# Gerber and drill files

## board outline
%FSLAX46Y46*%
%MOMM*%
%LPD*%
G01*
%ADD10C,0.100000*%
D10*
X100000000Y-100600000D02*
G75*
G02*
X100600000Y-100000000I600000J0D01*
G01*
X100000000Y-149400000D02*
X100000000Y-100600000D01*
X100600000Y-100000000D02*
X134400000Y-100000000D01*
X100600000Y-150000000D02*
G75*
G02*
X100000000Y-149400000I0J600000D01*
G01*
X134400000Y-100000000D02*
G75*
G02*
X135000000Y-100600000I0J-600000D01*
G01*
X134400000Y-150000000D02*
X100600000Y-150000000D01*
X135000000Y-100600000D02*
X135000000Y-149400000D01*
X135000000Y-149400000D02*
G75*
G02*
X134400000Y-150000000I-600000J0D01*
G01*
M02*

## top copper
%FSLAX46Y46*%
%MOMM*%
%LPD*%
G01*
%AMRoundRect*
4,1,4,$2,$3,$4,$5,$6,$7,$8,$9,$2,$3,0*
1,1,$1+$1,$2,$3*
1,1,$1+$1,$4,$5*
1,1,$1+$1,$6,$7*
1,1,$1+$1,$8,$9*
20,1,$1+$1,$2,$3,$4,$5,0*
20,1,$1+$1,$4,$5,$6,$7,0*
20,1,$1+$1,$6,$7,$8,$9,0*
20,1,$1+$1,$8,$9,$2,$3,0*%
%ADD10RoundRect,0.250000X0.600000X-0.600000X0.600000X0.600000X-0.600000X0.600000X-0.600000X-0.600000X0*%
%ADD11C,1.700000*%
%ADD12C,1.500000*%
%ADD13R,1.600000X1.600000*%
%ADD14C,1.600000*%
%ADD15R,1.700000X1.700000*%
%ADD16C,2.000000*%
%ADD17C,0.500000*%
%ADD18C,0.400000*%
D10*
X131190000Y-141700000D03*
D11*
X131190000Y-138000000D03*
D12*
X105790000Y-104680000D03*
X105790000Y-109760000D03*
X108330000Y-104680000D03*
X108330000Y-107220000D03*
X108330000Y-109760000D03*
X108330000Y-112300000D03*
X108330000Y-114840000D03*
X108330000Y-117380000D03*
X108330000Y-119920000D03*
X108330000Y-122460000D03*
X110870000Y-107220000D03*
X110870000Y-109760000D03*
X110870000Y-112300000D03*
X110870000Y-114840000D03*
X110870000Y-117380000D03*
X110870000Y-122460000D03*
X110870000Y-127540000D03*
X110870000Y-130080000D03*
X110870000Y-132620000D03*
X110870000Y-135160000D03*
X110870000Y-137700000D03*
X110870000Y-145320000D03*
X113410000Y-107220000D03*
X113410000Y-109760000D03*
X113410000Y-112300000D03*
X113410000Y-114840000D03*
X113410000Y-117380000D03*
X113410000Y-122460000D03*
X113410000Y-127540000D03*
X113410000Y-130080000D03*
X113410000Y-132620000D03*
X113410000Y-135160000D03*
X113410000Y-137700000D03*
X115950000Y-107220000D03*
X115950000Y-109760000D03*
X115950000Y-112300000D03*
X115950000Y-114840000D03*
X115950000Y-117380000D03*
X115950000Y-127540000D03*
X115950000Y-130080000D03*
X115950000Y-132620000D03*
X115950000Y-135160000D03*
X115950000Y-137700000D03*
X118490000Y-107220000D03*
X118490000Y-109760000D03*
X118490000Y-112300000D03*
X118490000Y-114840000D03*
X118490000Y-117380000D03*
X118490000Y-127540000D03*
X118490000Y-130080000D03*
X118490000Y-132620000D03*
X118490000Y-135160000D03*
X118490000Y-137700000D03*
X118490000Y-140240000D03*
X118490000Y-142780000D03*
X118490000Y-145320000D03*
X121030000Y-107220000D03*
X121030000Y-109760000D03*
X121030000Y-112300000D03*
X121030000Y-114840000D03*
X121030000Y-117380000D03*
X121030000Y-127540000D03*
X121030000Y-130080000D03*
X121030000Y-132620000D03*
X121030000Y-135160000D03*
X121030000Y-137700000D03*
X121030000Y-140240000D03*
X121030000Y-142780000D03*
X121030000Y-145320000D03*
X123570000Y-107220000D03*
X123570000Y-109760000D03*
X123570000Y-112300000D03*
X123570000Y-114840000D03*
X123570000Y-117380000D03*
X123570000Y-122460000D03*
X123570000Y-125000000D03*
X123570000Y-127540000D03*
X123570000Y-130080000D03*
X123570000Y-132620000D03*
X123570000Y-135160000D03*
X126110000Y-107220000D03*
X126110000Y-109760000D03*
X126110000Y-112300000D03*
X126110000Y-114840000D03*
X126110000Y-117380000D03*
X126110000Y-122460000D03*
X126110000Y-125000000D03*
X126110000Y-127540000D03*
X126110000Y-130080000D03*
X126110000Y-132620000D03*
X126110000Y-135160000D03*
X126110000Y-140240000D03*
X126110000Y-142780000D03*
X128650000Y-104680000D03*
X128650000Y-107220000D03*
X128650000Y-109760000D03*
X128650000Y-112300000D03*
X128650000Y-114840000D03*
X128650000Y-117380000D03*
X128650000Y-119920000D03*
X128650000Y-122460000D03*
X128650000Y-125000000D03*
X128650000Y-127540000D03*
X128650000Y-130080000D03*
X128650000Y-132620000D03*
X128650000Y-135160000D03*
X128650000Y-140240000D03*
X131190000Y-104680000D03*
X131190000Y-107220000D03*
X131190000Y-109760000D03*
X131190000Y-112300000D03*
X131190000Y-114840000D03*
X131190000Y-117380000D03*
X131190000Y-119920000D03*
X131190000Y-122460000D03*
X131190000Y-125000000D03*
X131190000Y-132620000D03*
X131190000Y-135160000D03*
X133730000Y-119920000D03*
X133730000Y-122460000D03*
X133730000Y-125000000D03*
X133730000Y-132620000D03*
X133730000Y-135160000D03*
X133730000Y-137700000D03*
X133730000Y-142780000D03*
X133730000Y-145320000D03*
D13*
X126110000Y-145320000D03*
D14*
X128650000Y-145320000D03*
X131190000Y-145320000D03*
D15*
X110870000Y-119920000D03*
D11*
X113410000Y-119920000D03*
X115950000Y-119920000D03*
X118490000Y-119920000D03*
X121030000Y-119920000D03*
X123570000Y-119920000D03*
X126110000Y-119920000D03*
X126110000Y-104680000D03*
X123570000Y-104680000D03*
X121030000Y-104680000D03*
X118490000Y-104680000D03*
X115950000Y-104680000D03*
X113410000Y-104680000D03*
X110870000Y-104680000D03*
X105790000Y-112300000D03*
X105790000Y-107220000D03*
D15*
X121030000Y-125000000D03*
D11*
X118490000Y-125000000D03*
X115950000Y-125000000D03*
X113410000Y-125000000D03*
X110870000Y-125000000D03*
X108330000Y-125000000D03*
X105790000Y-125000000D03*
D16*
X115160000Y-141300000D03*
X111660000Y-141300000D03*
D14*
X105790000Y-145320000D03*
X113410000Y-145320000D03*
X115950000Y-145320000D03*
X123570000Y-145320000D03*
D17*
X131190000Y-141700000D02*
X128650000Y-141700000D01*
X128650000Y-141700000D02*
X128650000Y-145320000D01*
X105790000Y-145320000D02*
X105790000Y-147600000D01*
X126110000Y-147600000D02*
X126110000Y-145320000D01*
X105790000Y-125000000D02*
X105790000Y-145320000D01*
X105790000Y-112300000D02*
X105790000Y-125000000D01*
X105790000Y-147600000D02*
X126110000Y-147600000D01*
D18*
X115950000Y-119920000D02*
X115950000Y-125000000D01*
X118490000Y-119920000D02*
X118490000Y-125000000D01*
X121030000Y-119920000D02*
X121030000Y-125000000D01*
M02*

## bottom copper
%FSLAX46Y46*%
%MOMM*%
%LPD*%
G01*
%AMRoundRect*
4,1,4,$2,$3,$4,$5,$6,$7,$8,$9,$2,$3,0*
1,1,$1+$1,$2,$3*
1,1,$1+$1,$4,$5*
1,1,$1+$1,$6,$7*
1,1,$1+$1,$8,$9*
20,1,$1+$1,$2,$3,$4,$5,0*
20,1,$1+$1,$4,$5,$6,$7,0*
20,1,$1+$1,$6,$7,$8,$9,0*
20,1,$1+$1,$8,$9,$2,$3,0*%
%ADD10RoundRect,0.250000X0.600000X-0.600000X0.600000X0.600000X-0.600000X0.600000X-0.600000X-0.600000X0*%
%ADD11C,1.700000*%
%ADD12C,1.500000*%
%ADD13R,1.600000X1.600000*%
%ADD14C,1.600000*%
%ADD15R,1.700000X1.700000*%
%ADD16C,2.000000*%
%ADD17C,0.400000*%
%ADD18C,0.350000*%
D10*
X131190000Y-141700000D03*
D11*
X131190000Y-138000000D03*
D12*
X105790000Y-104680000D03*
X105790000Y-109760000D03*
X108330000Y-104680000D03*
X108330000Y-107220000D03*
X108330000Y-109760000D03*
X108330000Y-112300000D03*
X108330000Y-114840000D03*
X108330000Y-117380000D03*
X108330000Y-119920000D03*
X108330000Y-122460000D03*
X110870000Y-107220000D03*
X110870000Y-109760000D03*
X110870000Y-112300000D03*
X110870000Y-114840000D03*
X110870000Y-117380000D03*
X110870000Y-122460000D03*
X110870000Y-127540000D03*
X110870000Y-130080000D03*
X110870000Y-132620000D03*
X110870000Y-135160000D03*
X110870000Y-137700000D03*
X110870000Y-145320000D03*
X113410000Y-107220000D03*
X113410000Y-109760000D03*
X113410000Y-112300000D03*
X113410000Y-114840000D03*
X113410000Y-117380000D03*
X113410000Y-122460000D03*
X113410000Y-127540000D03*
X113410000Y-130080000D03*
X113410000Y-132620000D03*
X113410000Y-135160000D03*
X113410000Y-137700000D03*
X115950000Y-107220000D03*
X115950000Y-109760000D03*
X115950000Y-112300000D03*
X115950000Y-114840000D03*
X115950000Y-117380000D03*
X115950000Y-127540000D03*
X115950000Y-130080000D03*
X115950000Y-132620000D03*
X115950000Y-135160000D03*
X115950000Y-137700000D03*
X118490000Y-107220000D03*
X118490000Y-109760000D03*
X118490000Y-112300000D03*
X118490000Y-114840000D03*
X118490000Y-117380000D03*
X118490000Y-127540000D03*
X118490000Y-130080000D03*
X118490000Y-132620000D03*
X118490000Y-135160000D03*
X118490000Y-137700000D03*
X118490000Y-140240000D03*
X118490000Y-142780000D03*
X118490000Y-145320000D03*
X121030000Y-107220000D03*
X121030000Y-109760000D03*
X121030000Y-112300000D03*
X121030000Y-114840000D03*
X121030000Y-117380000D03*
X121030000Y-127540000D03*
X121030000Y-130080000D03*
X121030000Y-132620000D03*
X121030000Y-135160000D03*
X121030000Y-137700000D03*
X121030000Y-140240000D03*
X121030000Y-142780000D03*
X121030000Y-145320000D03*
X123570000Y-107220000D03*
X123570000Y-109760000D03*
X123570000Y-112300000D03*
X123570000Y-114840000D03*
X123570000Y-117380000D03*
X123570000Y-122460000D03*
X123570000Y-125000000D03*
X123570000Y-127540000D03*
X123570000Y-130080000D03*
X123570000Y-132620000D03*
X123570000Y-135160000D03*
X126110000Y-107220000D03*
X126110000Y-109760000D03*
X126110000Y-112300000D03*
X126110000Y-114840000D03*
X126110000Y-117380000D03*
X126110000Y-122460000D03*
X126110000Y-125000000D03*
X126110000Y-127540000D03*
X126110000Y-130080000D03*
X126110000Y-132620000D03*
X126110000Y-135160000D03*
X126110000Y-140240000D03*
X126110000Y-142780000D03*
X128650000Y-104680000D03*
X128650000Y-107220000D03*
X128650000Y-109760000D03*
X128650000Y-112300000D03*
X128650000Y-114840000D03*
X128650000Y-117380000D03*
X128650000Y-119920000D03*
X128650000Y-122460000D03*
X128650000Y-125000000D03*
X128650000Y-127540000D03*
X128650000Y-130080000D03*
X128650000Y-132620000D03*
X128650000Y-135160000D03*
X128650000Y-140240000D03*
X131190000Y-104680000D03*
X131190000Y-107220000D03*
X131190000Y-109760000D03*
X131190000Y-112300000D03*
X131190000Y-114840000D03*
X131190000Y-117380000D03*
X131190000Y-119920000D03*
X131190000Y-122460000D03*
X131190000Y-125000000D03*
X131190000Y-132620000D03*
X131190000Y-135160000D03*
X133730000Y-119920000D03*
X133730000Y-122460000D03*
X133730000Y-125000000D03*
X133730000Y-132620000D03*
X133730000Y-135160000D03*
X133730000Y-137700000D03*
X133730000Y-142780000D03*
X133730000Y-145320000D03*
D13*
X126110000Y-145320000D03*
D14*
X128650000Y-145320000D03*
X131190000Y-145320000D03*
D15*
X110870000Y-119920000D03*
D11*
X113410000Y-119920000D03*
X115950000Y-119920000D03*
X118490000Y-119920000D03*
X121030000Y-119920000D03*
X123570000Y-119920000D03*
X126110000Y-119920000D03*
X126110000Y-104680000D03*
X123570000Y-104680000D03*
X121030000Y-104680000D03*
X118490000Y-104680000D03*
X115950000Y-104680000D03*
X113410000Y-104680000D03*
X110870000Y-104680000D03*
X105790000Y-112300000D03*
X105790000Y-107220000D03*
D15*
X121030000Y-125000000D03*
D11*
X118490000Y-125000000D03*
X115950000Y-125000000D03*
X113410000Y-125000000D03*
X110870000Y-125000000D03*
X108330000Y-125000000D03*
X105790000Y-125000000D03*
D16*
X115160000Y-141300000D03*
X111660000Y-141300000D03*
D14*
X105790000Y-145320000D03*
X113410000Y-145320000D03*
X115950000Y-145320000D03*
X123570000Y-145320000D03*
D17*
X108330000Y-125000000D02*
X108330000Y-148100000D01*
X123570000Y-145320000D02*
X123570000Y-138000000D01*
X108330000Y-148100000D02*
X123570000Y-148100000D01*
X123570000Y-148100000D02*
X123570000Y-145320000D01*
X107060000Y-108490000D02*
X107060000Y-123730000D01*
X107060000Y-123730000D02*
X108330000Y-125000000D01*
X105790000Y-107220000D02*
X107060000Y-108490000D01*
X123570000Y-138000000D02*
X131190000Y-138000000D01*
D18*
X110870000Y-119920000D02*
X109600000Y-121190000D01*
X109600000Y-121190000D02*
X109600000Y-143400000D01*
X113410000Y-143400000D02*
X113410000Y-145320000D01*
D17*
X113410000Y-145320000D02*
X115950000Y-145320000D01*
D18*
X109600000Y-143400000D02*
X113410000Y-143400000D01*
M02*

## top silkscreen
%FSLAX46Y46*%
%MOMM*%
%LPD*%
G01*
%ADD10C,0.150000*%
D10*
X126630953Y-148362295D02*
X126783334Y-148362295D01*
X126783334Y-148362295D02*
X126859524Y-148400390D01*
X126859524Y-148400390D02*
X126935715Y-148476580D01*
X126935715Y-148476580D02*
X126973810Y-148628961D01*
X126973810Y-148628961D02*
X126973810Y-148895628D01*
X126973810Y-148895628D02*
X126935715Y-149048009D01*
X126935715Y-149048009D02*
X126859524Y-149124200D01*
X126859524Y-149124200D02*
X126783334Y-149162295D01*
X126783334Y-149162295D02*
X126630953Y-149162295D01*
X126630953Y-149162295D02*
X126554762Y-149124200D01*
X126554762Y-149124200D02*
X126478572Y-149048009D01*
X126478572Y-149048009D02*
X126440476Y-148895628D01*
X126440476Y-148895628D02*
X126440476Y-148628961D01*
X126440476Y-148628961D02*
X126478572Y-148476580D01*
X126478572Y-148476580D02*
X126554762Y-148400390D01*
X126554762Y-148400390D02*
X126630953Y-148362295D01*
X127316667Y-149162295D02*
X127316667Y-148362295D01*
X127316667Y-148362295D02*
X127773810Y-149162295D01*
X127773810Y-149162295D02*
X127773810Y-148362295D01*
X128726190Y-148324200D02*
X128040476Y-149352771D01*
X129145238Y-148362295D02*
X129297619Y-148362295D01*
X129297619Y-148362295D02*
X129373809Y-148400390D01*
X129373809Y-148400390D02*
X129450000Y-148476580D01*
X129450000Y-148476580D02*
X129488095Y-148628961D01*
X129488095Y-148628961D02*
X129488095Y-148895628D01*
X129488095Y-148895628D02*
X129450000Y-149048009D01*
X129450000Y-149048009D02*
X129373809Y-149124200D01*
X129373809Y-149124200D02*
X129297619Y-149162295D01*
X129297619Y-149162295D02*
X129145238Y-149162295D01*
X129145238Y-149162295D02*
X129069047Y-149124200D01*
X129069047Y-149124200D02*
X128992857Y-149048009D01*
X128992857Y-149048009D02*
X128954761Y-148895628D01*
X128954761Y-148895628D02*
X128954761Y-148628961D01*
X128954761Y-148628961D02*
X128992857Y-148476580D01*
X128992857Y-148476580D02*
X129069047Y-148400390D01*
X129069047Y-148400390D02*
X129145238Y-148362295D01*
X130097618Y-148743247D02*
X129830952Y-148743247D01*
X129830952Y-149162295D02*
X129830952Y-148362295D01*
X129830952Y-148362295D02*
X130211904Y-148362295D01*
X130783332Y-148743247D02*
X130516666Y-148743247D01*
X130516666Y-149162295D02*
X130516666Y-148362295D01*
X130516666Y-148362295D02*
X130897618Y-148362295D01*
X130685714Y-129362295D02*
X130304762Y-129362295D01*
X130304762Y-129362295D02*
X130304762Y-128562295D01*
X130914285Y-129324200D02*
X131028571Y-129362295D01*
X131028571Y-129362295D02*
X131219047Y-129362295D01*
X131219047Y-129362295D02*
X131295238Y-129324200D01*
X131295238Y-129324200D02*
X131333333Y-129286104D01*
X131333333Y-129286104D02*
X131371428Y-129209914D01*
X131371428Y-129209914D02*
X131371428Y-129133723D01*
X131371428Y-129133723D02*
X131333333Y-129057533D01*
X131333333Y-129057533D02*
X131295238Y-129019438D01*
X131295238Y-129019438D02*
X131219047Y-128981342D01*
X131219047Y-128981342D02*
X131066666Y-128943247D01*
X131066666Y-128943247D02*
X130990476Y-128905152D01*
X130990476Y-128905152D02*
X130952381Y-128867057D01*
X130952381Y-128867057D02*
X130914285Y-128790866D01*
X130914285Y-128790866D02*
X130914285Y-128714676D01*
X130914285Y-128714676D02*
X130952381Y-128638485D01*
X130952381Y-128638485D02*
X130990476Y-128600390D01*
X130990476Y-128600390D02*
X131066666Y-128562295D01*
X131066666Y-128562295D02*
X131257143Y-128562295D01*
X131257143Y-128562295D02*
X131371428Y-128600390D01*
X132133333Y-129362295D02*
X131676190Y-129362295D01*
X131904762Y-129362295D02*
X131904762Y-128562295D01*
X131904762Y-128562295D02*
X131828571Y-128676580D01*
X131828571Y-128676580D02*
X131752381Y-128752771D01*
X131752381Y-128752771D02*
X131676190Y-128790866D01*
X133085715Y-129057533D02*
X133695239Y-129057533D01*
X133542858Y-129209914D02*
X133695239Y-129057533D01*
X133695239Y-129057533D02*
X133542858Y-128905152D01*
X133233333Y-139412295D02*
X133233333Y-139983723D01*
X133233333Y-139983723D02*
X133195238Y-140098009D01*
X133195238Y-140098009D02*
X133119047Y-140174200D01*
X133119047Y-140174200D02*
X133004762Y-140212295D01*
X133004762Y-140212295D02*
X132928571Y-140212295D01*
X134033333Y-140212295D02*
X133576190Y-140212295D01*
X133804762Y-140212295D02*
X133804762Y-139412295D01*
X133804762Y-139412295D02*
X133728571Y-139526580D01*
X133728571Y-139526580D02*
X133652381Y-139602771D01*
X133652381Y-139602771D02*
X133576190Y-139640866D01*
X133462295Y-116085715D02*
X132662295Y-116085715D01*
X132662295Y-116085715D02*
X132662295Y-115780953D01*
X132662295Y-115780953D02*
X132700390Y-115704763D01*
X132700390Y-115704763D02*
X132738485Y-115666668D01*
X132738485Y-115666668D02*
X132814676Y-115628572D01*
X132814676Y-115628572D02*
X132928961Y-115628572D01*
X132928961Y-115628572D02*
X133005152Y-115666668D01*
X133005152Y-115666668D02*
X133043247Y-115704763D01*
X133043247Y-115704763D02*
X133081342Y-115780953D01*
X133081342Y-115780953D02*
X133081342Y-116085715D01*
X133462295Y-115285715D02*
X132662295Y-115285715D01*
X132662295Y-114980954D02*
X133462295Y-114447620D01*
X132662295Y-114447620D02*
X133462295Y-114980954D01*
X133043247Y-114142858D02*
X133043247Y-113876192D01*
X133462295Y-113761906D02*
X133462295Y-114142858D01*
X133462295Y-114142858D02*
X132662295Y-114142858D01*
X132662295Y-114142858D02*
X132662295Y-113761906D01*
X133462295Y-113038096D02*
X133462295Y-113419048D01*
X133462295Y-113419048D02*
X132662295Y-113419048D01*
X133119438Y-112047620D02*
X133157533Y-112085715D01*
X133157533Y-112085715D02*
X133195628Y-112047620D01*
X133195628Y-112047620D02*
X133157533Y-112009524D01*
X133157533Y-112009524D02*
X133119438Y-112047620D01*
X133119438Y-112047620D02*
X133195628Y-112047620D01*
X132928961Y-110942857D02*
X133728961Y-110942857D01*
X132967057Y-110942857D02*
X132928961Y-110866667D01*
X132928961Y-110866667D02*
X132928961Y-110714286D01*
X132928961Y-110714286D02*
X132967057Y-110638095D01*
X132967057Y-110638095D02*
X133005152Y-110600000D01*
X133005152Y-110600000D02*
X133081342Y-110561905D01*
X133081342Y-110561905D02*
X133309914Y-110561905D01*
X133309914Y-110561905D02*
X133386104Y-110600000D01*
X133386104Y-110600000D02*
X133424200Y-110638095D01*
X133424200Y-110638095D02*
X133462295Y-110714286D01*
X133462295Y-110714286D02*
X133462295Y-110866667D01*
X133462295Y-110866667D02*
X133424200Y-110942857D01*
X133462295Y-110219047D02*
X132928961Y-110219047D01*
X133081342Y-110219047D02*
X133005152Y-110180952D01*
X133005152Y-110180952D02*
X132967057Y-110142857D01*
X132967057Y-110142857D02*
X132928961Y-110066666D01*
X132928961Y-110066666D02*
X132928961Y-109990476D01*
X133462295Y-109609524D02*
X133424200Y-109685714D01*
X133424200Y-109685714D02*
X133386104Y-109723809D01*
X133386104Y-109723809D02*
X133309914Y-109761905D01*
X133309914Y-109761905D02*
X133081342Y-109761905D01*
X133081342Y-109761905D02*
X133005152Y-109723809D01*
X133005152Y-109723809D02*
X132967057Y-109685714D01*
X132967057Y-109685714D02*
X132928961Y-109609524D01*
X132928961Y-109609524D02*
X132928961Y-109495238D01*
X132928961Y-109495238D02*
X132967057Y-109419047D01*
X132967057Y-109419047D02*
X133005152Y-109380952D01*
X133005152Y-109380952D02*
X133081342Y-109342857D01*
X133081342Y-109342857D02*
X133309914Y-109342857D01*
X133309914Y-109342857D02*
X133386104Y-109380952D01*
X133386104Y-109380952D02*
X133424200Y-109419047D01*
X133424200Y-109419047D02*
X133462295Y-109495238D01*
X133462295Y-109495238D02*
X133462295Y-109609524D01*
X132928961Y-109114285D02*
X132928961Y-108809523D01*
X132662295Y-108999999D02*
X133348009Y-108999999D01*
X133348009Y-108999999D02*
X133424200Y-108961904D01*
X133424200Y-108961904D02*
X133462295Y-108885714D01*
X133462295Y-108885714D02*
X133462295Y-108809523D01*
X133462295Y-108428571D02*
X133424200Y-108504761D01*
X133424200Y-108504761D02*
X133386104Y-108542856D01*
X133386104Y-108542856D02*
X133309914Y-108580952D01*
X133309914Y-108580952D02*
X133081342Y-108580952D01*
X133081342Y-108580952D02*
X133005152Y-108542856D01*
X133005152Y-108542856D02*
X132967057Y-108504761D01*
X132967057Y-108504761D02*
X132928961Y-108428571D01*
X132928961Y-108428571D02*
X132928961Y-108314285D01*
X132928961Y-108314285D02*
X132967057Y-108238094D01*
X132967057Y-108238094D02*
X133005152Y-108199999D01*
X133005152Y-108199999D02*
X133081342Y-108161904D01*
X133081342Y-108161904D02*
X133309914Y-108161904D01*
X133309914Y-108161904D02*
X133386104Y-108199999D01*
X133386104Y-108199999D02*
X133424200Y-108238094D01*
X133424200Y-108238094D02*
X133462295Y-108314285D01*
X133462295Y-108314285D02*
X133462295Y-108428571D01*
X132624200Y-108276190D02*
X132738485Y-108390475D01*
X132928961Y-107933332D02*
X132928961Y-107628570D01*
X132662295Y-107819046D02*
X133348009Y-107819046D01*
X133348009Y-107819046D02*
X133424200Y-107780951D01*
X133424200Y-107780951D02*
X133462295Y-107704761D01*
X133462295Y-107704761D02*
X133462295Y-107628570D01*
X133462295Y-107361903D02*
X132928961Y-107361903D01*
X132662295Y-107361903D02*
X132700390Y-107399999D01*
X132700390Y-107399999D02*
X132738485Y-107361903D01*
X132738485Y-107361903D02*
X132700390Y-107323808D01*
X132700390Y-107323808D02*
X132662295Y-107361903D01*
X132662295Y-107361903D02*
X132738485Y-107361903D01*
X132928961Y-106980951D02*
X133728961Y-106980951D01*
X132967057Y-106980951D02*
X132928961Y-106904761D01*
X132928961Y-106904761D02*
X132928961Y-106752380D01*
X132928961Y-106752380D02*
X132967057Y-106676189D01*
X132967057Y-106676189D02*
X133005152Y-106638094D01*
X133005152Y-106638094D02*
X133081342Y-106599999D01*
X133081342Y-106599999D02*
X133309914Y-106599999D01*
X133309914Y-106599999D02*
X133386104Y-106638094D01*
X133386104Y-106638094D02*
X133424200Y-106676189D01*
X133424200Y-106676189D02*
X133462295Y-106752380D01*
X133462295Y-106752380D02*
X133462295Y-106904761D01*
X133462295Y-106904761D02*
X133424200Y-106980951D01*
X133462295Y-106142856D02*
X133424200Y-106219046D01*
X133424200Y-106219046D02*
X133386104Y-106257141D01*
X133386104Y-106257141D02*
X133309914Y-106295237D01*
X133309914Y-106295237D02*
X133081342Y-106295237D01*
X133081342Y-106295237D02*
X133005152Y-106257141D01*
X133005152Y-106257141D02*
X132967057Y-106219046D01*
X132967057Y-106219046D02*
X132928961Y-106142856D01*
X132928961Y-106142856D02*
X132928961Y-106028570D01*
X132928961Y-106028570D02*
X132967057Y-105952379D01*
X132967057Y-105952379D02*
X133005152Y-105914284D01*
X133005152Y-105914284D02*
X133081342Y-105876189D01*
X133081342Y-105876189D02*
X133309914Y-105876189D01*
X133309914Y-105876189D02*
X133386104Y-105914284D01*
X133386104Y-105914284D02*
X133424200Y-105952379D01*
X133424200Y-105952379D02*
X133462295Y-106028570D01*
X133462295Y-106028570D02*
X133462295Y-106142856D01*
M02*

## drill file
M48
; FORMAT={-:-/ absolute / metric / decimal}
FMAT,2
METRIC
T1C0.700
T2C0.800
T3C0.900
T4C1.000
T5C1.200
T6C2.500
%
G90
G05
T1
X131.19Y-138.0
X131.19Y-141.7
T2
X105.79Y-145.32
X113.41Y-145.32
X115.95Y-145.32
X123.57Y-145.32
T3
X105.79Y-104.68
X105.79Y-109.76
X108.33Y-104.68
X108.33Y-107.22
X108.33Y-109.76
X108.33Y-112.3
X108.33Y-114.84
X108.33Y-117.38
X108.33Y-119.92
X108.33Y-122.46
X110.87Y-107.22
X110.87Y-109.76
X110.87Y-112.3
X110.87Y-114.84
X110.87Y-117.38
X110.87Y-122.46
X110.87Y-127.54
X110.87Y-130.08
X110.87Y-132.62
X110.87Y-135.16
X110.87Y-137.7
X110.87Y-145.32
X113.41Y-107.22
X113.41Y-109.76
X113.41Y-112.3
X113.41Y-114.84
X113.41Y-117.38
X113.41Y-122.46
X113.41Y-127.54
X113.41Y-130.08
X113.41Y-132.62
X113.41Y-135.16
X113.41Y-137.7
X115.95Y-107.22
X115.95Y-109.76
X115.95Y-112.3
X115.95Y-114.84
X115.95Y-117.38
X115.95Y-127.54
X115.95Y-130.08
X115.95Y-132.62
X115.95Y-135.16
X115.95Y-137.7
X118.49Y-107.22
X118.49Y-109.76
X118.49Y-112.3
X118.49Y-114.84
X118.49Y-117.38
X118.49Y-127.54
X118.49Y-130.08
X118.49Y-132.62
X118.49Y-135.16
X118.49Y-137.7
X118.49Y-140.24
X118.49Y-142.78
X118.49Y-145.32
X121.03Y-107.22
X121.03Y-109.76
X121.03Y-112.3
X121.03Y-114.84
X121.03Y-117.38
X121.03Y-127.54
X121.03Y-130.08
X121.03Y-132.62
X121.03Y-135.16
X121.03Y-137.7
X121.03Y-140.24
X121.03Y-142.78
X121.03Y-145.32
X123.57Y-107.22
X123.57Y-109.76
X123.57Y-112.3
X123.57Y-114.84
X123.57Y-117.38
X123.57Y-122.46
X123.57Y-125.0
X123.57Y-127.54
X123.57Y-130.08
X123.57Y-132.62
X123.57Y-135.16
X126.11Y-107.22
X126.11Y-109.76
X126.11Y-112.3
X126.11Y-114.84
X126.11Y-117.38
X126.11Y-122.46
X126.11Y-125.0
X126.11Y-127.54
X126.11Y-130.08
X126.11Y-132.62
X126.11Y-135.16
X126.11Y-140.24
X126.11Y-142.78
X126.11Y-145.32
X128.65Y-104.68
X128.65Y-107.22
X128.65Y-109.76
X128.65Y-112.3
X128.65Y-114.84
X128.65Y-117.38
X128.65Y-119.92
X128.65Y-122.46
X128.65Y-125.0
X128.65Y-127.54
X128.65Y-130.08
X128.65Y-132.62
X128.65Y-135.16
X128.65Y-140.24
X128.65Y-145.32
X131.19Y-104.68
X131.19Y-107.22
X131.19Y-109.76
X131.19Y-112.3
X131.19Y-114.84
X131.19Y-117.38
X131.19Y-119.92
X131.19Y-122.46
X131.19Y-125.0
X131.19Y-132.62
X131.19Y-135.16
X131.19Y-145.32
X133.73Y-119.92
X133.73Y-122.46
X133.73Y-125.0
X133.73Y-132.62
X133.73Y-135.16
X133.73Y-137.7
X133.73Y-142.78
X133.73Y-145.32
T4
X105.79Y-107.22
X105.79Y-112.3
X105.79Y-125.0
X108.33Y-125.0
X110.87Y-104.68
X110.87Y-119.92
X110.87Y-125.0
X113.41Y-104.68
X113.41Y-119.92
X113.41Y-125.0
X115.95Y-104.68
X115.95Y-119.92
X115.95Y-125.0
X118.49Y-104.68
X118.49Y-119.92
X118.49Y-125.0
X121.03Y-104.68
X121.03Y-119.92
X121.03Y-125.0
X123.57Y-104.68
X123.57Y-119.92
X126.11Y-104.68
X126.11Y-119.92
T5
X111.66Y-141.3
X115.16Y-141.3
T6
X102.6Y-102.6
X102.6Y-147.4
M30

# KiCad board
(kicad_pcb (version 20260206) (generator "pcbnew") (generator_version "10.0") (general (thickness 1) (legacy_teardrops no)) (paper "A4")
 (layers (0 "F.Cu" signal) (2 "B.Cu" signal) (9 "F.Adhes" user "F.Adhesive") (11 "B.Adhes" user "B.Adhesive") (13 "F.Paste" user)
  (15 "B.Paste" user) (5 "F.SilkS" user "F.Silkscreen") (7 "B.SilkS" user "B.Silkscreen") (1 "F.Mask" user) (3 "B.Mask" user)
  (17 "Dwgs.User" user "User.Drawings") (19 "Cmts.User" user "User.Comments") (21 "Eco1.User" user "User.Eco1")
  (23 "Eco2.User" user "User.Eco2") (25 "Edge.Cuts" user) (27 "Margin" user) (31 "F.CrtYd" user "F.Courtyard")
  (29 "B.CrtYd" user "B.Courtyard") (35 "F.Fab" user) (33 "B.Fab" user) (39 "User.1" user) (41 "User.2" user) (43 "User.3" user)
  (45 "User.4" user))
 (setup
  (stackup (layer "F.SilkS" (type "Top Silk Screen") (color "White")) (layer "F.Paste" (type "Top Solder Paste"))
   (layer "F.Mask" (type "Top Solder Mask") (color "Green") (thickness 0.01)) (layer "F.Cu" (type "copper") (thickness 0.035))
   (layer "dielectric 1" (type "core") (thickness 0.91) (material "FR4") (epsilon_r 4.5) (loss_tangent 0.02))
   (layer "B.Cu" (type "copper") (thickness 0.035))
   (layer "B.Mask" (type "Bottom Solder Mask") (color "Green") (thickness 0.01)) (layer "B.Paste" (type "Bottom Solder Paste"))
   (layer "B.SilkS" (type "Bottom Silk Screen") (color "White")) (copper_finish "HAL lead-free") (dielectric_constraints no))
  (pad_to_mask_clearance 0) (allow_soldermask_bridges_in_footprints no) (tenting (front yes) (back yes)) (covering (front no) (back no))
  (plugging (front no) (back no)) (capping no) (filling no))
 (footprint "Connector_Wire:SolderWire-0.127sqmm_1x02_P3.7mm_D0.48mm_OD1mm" (layer "F.Cu") (at 131.19 141.7 90)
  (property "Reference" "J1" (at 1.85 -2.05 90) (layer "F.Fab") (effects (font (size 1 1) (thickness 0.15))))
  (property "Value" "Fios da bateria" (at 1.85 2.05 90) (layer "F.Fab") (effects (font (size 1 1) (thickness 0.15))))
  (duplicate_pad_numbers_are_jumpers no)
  (pad "1" thru_hole roundrect (at 0 0 90) (size 1.7 1.7) (drill 0.7) (layers "*.Cu" "*.Mask") (remove_unused_layers no)
   (roundrect_rratio 0.147059) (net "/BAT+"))
  (pad "2" thru_hole circle (at 3.7 0 90) (size 1.7 1.7) (drill 0.7) (layers "*.Cu" "*.Mask") (remove_unused_layers no) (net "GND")))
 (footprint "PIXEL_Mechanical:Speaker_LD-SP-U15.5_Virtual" (layer "F.Cu") (at 143.7 129)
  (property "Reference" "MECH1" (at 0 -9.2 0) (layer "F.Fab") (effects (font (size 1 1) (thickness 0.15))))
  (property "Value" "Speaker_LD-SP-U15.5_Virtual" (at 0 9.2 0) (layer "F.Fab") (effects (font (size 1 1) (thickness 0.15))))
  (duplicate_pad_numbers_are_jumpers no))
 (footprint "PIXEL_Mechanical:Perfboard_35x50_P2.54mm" (layer "F.Cu") (at 0 0)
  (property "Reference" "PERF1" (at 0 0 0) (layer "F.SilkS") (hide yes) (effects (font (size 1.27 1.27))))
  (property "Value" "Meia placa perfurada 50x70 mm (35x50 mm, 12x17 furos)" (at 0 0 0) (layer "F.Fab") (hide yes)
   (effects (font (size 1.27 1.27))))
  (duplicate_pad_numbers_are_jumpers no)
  (pad "" np_thru_hole circle (at 102.6 102.6) (size 2.5 2.5) (drill 2.5) (layers "*.Cu" "*.Mask"))
  (pad "" np_thru_hole circle (at 102.6 147.4) (size 2.5 2.5) (drill 2.5) (layers "*.Cu" "*.Mask"))
  (pad "" thru_hole circle (at 105.79 104.68) (size 1.5 1.5) (drill 0.9) (layers "*.Cu" "*.Mask") (remove_unused_layers no))
  (pad "" thru_hole circle (at 105.79 109.76) (size 1.5 1.5) (drill 0.9) (layers "*.Cu" "*.Mask") (remove_unused_layers no))
  (pad "" thru_hole circle (at 108.33 104.68) (size 1.5 1.5) (drill 0.9) (layers "*.Cu" "*.Mask") (remove_unused_layers no))
  (pad "" thru_hole circle (at 108.33 107.22) (size 1.5 1.5) (drill 0.9) (layers "*.Cu" "*.Mask") (remove_unused_layers no))
  (pad "" thru_hole circle (at 108.33 109.76) (size 1.5 1.5) (drill 0.9) (layers "*.Cu" "*.Mask") (remove_unused_layers no))
  (pad "" thru_hole circle (at 108.33 112.3) (size 1.5 1.5) (drill 0.9) (layers "*.Cu" "*.Mask") (remove_unused_layers no))
  (pad "" thru_hole circle (at 108.33 114.84) (size 1.5 1.5) (drill 0.9) (layers "*.Cu" "*.Mask") (remove_unused_layers no))
  (pad "" thru_hole circle (at 108.33 117.38) (size 1.5 1.5) (drill 0.9) (layers "*.Cu" "*.Mask") (remove_unused_layers no))
  (pad "" thru_hole circle (at 108.33 119.92) (size 1.5 1.5) (drill 0.9) (layers "*.Cu" "*.Mask") (remove_unused_layers no))
  (pad "" thru_hole circle (at 108.33 122.46) (size 1.5 1.5) (drill 0.9) (layers "*.Cu" "*.Mask") (remove_unused_layers no))
  (pad "" thru_hole circle (at 110.87 107.22) (size 1.5 1.5) (drill 0.9) (layers "*.Cu" "*.Mask") (remove_unused_layers no))
  (pad "" thru_hole circle (at 110.87 109.76) (size 1.5 1.5) (drill 0.9) (layers "*.Cu" "*.Mask") (remove_unused_layers no))
  (pad "" thru_hole circle (at 110.87 112.3) (size 1.5 1.5) (drill 0.9) (layers "*.Cu" "*.Mask") (remove_unused_layers no))
  (pad "" thru_hole circle (at 110.87 114.84) (size 1.5 1.5) (drill 0.9) (layers "*.Cu" "*.Mask") (remove_unused_layers no))
  (pad "" thru_hole circle (at 110.87 117.38) (size 1.5 1.5) (drill 0.9) (layers "*.Cu" "*.Mask") (remove_unused_layers no))
  (pad "" thru_hole circle (at 110.87 122.46) (size 1.5 1.5) (drill 0.9) (layers "*.Cu" "*.Mask") (remove_unused_layers no))
  (pad "" thru_hole circle (at 110.87 127.54) (size 1.5 1.5) (drill 0.9) (layers "*.Cu" "*.Mask") (remove_unused_layers no))
  (pad "" thru_hole circle (at 110.87 130.08) (size 1.5 1.5) (drill 0.9) (layers "*.Cu" "*.Mask") (remove_unused_layers no))
  (pad "" thru_hole circle (at 110.87 132.62) (size 1.5 1.5) (drill 0.9) (layers "*.Cu" "*.Mask") (remove_unused_layers no))
  (pad "" thru_hole circle (at 110.87 135.16) (size 1.5 1.5) (drill 0.9) (layers "*.Cu" "*.Mask") (remove_unused_layers no))
  (pad "" thru_hole circle (at 110.87 137.7) (size 1.5 1.5) (drill 0.9) (layers "*.Cu" "*.Mask") (remove_unused_layers no))
  (pad "" thru_hole circle (at 110.87 145.32) (size 1.5 1.5) (drill 0.9) (layers "*.Cu" "*.Mask") (remove_unused_layers no))
  (pad "" thru_hole circle (at 113.41 107.22) (size 1.5 1.5) (drill 0.9) (layers "*.Cu" "*.Mask") (remove_unused_layers no))
  (pad "" thru_hole circle (at 113.41 109.76) (size 1.5 1.5) (drill 0.9) (layers "*.Cu" "*.Mask") (remove_unused_layers no))
  (pad "" thru_hole circle (at 113.41 112.3) (size 1.5 1.5) (drill 0.9) (layers "*.Cu" "*.Mask") (remove_unused_layers no))
  (pad "" thru_hole circle (at 113.41 114.84) (size 1.5 1.5) (drill 0.9) (layers "*.Cu" "*.Mask") (remove_unused_layers no))
  (pad "" thru_hole circle (at 113.41 117.38) (size 1.5 1.5) (drill 0.9) (layers "*.Cu" "*.Mask") (remove_unused_layers no))
  (pad "" thru_hole circle (at 113.41 122.46) (size 1.5 1.5) (drill 0.9) (layers "*.Cu" "*.Mask") (remove_unused_layers no))
  (pad "" thru_hole circle (at 113.41 127.54) (size 1.5 1.5) (drill 0.9) (layers "*.Cu" "*.Mask") (remove_unused_layers no))
  (pad "" thru_hole circle (at 113.41 130.08) (size 1.5 1.5) (drill 0.9) (layers "*.Cu" "*.Mask") (remove_unused_layers no))
  (pad "" thru_hole circle (at 113.41 132.62) (size 1.5 1.5) (drill 0.9) (layers "*.Cu" "*.Mask") (remove_unused_layers no))
  (pad "" thru_hole circle (at 113.41 135.16) (size 1.5 1.5) (drill 0.9) (layers "*.Cu" "*.Mask") (remove_unused_layers no))
  (pad "" thru_hole circle (at 113.41 137.7) (size 1.5 1.5) (drill 0.9) (layers "*.Cu" "*.Mask") (remove_unused_layers no))
  (pad "" thru_hole circle (at 115.95 107.22) (size 1.5 1.5) (drill 0.9) (layers "*.Cu" "*.Mask") (remove_unused_layers no))
  (pad "" thru_hole circle (at 115.95 109.76) (size 1.5 1.5) (drill 0.9) (layers "*.Cu" "*.Mask") (remove_unused_layers no))
  (pad "" thru_hole circle (at 115.95 112.3) (size 1.5 1.5) (drill 0.9) (layers "*.Cu" "*.Mask") (remove_unused_layers no))
  (pad "" thru_hole circle (at 115.95 114.84) (size 1.5 1.5) (drill 0.9) (layers "*.Cu" "*.Mask") (remove_unused_layers no))
  (pad "" thru_hole circle (at 115.95 117.38) (size 1.5 1.5) (drill 0.9) (layers "*.Cu" "*.Mask") (remove_unused_layers no))
  (pad "" thru_hole circle (at 115.95 127.54) (size 1.5 1.5) (drill 0.9) (layers "*.Cu" "*.Mask") (remove_unused_layers no))
  (pad "" thru_hole circle (at 115.95 130.08) (size 1.5 1.5) (drill 0.9) (layers "*.Cu" "*.Mask") (remove_unused_layers no))
  (pad "" thru_hole circle (at 115.95 132.62) (size 1.5 1.5) (drill 0.9) (layers "*.Cu" "*.Mask") (remove_unused_layers no))
  (pad "" thru_hole circle (at 115.95 135.16) (size 1.5 1.5) (drill 0.9) (layers "*.Cu" "*.Mask") (remove_unused_layers no))
  (pad "" thru_hole circle (at 115.95 137.7) (size 1.5 1.5) (drill 0.9) (layers "*.Cu" "*.Mask") (remove_unused_layers no))
  (pad "" thru_hole circle (at 118.49 107.22) (size 1.5 1.5) (drill 0.9) (layers "*.Cu" "*.Mask") (remove_unused_layers no))
  (pad "" thru_hole circle (at 118.49 109.76) (size 1.5 1.5) (drill 0.9) (layers "*.Cu" "*.Mask") (remove_unused_layers no))
  (pad "" thru_hole circle (at 118.49 112.3) (size 1.5 1.5) (drill 0.9) (layers "*.Cu" "*.Mask") (remove_unused_layers no))
  (pad "" thru_hole circle (at 118.49 114.84) (size 1.5 1.5) (drill 0.9) (layers "*.Cu" "*.Mask") (remove_unused_layers no))
  (pad "" thru_hole circle (at 118.49 117.38) (size 1.5 1.5) (drill 0.9) (layers "*.Cu" "*.Mask") (remove_unused_layers no))
  (pad "" thru_hole circle (at 118.49 127.54) (size 1.5 1.5) (drill 0.9) (layers "*.Cu" "*.Mask") (remove_unused_layers no))
  (pad "" thru_hole circle (at 118.49 130.08) (size 1.5 1.5) (drill 0.9) (layers "*.Cu" "*.Mask") (remove_unused_layers no))
  (pad "" thru_hole circle (at 118.49 132.62) (size 1.5 1.5) (drill 0.9) (layers "*.Cu" "*.Mask") (remove_unused_layers no))
  (pad "" thru_hole circle (at 118.49 135.16) (size 1.5 1.5) (drill 0.9) (layers "*.Cu" "*.Mask") (remove_unused_layers no))
  (pad "" thru_hole circle (at 118.49 137.7) (size 1.5 1.5) (drill 0.9) (layers "*.Cu" "*.Mask") (remove_unused_layers no))
  (pad "" thru_hole circle (at 118.49 140.24) (size 1.5 1.5) (drill 0.9) (layers "*.Cu" "*.Mask") (remove_unused_layers no))
  (pad "" thru_hole circle (at 118.49 142.78) (size 1.5 1.5) (drill 0.9) (layers "*.Cu" "*.Mask") (remove_unused_layers no))
  (pad "" thru_hole circle (at 118.49 145.32) (size 1.5 1.5) (drill 0.9) (layers "*.Cu" "*.Mask") (remove_unused_layers no))
  (pad "" thru_hole circle (at 121.03 107.22) (size 1.5 1.5) (drill 0.9) (layers "*.Cu" "*.Mask") (remove_unused_layers no))
  (pad "" thru_hole circle (at 121.03 109.76) (size 1.5 1.5) (drill 0.9) (layers "*.Cu" "*.Mask") (remove_unused_layers no))
  (pad "" thru_hole circle (at 121.03 112.3) (size 1.5 1.5) (drill 0.9) (layers "*.Cu" "*.Mask") (remove_unused_layers no))
  (pad "" thru_hole circle (at 121.03 114.84) (size 1.5 1.5) (drill 0.9) (layers "*.Cu" "*.Mask") (remove_unused_layers no))
  (pad "" thru_hole circle (at 121.03 117.38) (size 1.5 1.5) (drill 0.9) (layers "*.Cu" "*.Mask") (remove_unused_layers no))
  (pad "" thru_hole circle (at 121.03 127.54) (size 1.5 1.5) (drill 0.9) (layers "*.Cu" "*.Mask") (remove_unused_layers no))
  (pad "" thru_hole circle (at 121.03 130.08) (size 1.5 1.5) (drill 0.9) (layers "*.Cu" "*.Mask") (remove_unused_layers no))
  (pad "" thru_hole circle (at 121.03 132.62) (size 1.5 1.5) (drill 0.9) (layers "*.Cu" "*.Mask") (remove_unused_layers no))
  (pad "" thru_hole circle (at 121.03 135.16) (size 1.5 1.5) (drill 0.9) (layers "*.Cu" "*.Mask") (remove_unused_layers no))
  (pad "" thru_hole circle (at 121.03 137.7) (size 1.5 1.5) (drill 0.9) (layers "*.Cu" "*.Mask") (remove_unused_layers no))
  (pad "" thru_hole circle (at 121.03 140.24) (size 1.5 1.5) (drill 0.9) (layers "*.Cu" "*.Mask") (remove_unused_layers no))
  (pad "" thru_hole circle (at 121.03 142.78) (size 1.5 1.5) (drill 0.9) (layers "*.Cu" "*.Mask") (remove_unused_layers no))
  (pad "" thru_hole circle (at 121.03 145.32) (size 1.5 1.5) (drill 0.9) (layers "*.Cu" "*.Mask") (remove_unused_layers no))
  (pad "" thru_hole circle (at 123.57 107.22) (size 1.5 1.5) (drill 0.9) (layers "*.Cu" "*.Mask") (remove_unused_layers no))
  (pad "" thru_hole circle (at 123.57 109.76) (size 1.5 1.5) (drill 0.9) (layers "*.Cu" "*.Mask") (remove_unused_layers no))
  (pad "" thru_hole circle (at 123.57 112.3) (size 1.5 1.5) (drill 0.9) (layers "*.Cu" "*.Mask") (remove_unused_layers no))
  (pad "" thru_hole circle (at 123.57 114.84) (size 1.5 1.5) (drill 0.9) (layers "*.Cu" "*.Mask") (remove_unused_layers no))
  (pad "" thru_hole circle (at 123.57 117.38) (size 1.5 1.5) (drill 0.9) (layers "*.Cu" "*.Mask") (remove_unused_layers no))
  (pad "" thru_hole circle (at 123.57 122.46) (size 1.5 1.5) (drill 0.9) (layers "*.Cu" "*.Mask") (remove_unused_layers no))
  (pad "" thru_hole circle (at 123.57 125) (size 1.5 1.5) (drill 0.9) (layers "*.Cu" "*.Mask") (remove_unused_layers no))
  (pad "" thru_hole circle (at 123.57 127.54) (size 1.5 1.5) (drill 0.9) (layers "*.Cu" "*.Mask") (remove_unused_layers no))
  (pad "" thru_hole circle (at 123.57 130.08) (size 1.5 1.5) (drill 0.9) (layers "*.Cu" "*.Mask") (remove_unused_layers no))
  (pad "" thru_hole circle (at 123.57 132.62) (size 1.5 1.5) (drill 0.9) (layers "*.Cu" "*.Mask") (remove_unused_layers no))
  (pad "" thru_hole circle (at 123.57 135.16) (size 1.5 1.5) (drill 0.9) (layers "*.Cu" "*.Mask") (remove_unused_layers no))
  (pad "" thru_hole circle (at 126.11 107.22) (size 1.5 1.5) (drill 0.9) (layers "*.Cu" "*.Mask") (remove_unused_layers no))
  (pad "" thru_hole circle (at 126.11 109.76) (size 1.5 1.5) (drill 0.9) (layers "*.Cu" "*.Mask") (remove_unused_layers no))
  (pad "" thru_hole circle (at 126.11 112.3) (size 1.5 1.5) (drill 0.9) (layers "*.Cu" "*.Mask") (remove_unused_layers no))
  (pad "" thru_hole circle (at 126.11 114.84) (size 1.5 1.5) (drill 0.9) (layers "*.Cu" "*.Mask") (remove_unused_layers no))
  (pad "" thru_hole circle (at 126.11 117.38) (size 1.5 1.5) (drill 0.9) (layers "*.Cu" "*.Mask") (remove_unused_layers no))
  (pad "" thru_hole circle (at 126.11 122.46) (size 1.5 1.5) (drill 0.9) (layers "*.Cu" "*.Mask") (remove_unused_layers no))
  (pad "" thru_hole circle (at 126.11 125) (size 1.5 1.5) (drill 0.9) (layers "*.Cu" "*.Mask") (remove_unused_layers no))
  (pad "" thru_hole circle (at 126.11 127.54) (size 1.5 1.5) (drill 0.9) (layers "*.Cu" "*.Mask") (remove_unused_layers no))
  (pad "" thru_hole circle (at 126.11 130.08) (size 1.5 1.5) (drill 0.9) (layers "*.Cu" "*.Mask") (remove_unused_layers no))
  (pad "" thru_hole circle (at 126.11 132.62) (size 1.5 1.5) (drill 0.9) (layers "*.Cu" "*.Mask") (remove_unused_layers no))
  (pad "" thru_hole circle (at 126.11 135.16) (size 1.5 1.5) (drill 0.9) (layers "*.Cu" "*.Mask") (remove_unused_layers no))
  (pad "" thru_hole circle (at 126.11 140.24) (size 1.5 1.5) (drill 0.9) (layers "*.Cu" "*.Mask") (remove_unused_layers no))
  (pad "" thru_hole circle (at 126.11 142.78) (size 1.5 1.5) (drill 0.9) (layers "*.Cu" "*.Mask") (remove_unused_layers no))
  (pad "" thru_hole circle (at 128.65 104.68) (size 1.5 1.5) (drill 0.9) (layers "*.Cu" "*.Mask") (remove_unused_layers no))
  (pad "" thru_hole circle (at 128.65 107.22) (size 1.5 1.5) (drill 0.9) (layers "*.Cu" "*.Mask") (remove_unused_layers no))
  (pad "" thru_hole circle (at 128.65 109.76) (size 1.5 1.5) (drill 0.9) (layers "*.Cu" "*.Mask") (remove_unused_layers no))
  (pad "" thru_hole circle (at 128.65 112.3) (size 1.5 1.5) (drill 0.9) (layers "*.Cu" "*.Mask") (remove_unused_layers no))
  (pad "" thru_hole circle (at 128.65 114.84) (size 1.5 1.5) (drill 0.9) (layers "*.Cu" "*.Mask") (remove_unused_layers no))
  (pad "" thru_hole circle (at 128.65 117.38) (size 1.5 1.5) (drill 0.9) (layers "*.Cu" "*.Mask") (remove_unused_layers no))
  (pad "" thru_hole circle (at 128.65 119.92) (size 1.5 1.5) (drill 0.9) (layers "*.Cu" "*.Mask") (remove_unused_layers no))
  (pad "" thru_hole circle (at 128.65 122.46) (size 1.5 1.5) (drill 0.9) (layers "*.Cu" "*.Mask") (remove_unused_layers no))
  (pad "" thru_hole circle (at 128.65 125) (size 1.5 1.5) (drill 0.9) (layers "*.Cu" "*.Mask") (remove_unused_layers no))
  (pad "" thru_hole circle (at 128.65 127.54) (size 1.5 1.5) (drill 0.9) (layers "*.Cu" "*.Mask") (remove_unused_layers no))
  (pad "" thru_hole circle (at 128.65 130.08) (size 1.5 1.5) (drill 0.9) (layers "*.Cu" "*.Mask") (remove_unused_layers no))
  (pad "" thru_hole circle (at 128.65 132.62) (size 1.5 1.5) (drill 0.9) (layers "*.Cu" "*.Mask") (remove_unused_layers no))
  (pad "" thru_hole circle (at 128.65 135.16) (size 1.5 1.5) (drill 0.9) (layers "*.Cu" "*.Mask") (remove_unused_layers no))
  (pad "" thru_hole circle (at 128.65 140.24) (size 1.5 1.5) (drill 0.9) (layers "*.Cu" "*.Mask") (remove_unused_layers no))
  (pad "" thru_hole circle (at 131.19 104.68) (size 1.5 1.5) (drill 0.9) (layers "*.Cu" "*.Mask") (remove_unused_layers no))
  (pad "" thru_hole circle (at 131.19 107.22) (size 1.5 1.5) (drill 0.9) (layers "*.Cu" "*.Mask") (remove_unused_layers no))
  (pad "" thru_hole circle (at 131.19 109.76) (size 1.5 1.5) (drill 0.9) (layers "*.Cu" "*.Mask") (remove_unused_layers no))
  (pad "" thru_hole circle (at 131.19 112.3) (size 1.5 1.5) (drill 0.9) (layers "*.Cu" "*.Mask") (remove_unused_layers no))
  (pad "" thru_hole circle (at 131.19 114.84) (size 1.5 1.5) (drill 0.9) (layers "*.Cu" "*.Mask") (remove_unused_layers no))
  (pad "" thru_hole circle (at 131.19 117.38) (size 1.5 1.5) (drill 0.9) (layers "*.Cu" "*.Mask") (remove_unused_layers no))
  (pad "" thru_hole circle (at 131.19 119.92) (size 1.5 1.5) (drill 0.9) (layers "*.Cu" "*.Mask") (remove_unused_layers no))
  (pad "" thru_hole circle (at 131.19 122.46) (size 1.5 1.5) (drill 0.9) (layers "*.Cu" "*.Mask") (remove_unused_layers no))
  (pad "" thru_hole circle (at 131.19 125) (size 1.5 1.5) (drill 0.9) (layers "*.Cu" "*.Mask") (remove_unused_layers no))
  (pad "" thru_hole circle (at 131.19 132.62) (size 1.5 1.5) (drill 0.9) (layers "*.Cu" "*.Mask") (remove_unused_layers no))
  (pad "" thru_hole circle (at 131.19 135.16) (size 1.5 1.5) (drill 0.9) (layers "*.Cu" "*.Mask") (remove_unused_layers no))
  (pad "" thru_hole circle (at 133.73 119.92) (size 1.5 1.5) (drill 0.9) (layers "*.Cu" "*.Mask") (remove_unused_layers no))
  (pad "" thru_hole circle (at 133.73 122.46) (size 1.5 1.5) (drill 0.9) (layers "*.Cu" "*.Mask") (remove_unused_layers no))
  (pad "" thru_hole circle (at 133.73 125) (size 1.5 1.5) (drill 0.9) (layers "*.Cu" "*.Mask") (remove_unused_layers no))
  (pad "" thru_hole circle (at 133.73 132.62) (size 1.5 1.5) (drill 0.9) (layers "*.Cu" "*.Mask") (remove_unused_layers no))
  (pad "" thru_hole circle (at 133.73 135.16) (size 1.5 1.5) (drill 0.9) (layers "*.Cu" "*.Mask") (remove_unused_layers no))
  (pad "" thru_hole circle (at 133.73 137.7) (size 1.5 1.5) (drill 0.9) (layers "*.Cu" "*.Mask") (remove_unused_layers no))
  (pad "" thru_hole circle (at 133.73 142.78) (size 1.5 1.5) (drill 0.9) (layers "*.Cu" "*.Mask") (remove_unused_layers no))
  (pad "" thru_hole circle (at 133.73 145.32) (size 1.5 1.5) (drill 0.9) (layers "*.Cu" "*.Mask") (remove_unused_layers no)))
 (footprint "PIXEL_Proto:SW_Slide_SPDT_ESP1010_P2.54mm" (layer "F.Cu") (at 128.65 145.32)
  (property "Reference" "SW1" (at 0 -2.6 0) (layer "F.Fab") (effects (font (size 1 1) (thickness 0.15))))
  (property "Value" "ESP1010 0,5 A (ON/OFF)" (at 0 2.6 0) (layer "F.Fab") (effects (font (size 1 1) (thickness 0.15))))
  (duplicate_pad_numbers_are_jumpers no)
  (pad "1" thru_hole rect (at -2.54 0) (size 1.6 1.6) (drill 0.9) (layers "*.Cu" "*.Mask") (remove_unused_layers no) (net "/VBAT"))
  (pad "2" thru_hole circle (at 0 0) (size 1.6 1.6) (drill 0.9) (layers "*.Cu" "*.Mask") (remove_unused_layers no) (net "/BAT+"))
  (pad "3" thru_hole circle (at 2.54 0) (size 1.6 1.6) (drill 0.9) (layers "*.Cu" "*.Mask") (remove_unused_layers no)
   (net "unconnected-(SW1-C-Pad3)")))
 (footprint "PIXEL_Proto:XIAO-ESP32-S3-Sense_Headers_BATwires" (layer "F.Cu") (at 118.49 112.3 180)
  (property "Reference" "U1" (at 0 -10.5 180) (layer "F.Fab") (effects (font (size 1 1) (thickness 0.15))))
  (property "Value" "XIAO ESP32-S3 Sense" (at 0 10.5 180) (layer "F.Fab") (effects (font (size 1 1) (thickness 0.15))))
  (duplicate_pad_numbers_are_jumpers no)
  (pad "1" thru_hole rect (at 7.62 -7.62 180) (size 1.7 1.7) (drill 1) (layers "*.Cu" "*.Mask") (remove_unused_layers no)
   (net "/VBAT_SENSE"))
  (pad "2" thru_hole circle (at 5.08 -7.62 180) (size 1.7 1.7) (drill 1) (layers "*.Cu" "*.Mask") (remove_unused_layers no)
   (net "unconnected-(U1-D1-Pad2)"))
  (pad "3" thru_hole circle (at 2.54 -7.62 180) (size 1.7 1.7) (drill 1) (layers "*.Cu" "*.Mask") (remove_unused_layers no)
   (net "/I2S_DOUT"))
  (pad "4" thru_hole circle (at 0 -7.62 180) (size 1.7 1.7) (drill 1) (layers "*.Cu" "*.Mask") (remove_unused_layers no) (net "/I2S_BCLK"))
  (pad "5" thru_hole circle (at -2.54 -7.62 180) (size 1.7 1.7) (drill 1) (layers "*.Cu" "*.Mask") (remove_unused_layers no)
   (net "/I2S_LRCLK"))
  (pad "6" thru_hole circle (at -5.08 -7.62 180) (size 1.7 1.7) (drill 1) (layers "*.Cu" "*.Mask") (remove_unused_layers no)
   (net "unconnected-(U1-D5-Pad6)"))
  (pad "7" thru_hole circle (at -7.62 -7.62 180) (size 1.7 1.7) (drill 1) (layers "*.Cu" "*.Mask") (remove_unused_layers no)
   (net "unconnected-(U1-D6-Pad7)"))
  (pad "8" thru_hole circle (at -7.62 7.62 180) (size 1.7 1.7) (drill 1) (layers "*.Cu" "*.Mask") (remove_unused_layers no)
   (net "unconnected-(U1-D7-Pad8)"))
  (pad "9" thru_hole circle (at -5.08 7.62 180) (size 1.7 1.7) (drill 1) (layers "*.Cu" "*.Mask") (remove_unused_layers no)
   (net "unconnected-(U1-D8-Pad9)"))
  (pad "10" thru_hole circle (at -2.54 7.62 180) (size 1.7 1.7) (drill 1) (layers "*.Cu" "*.Mask") (remove_unused_layers no)
   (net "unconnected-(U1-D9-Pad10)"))
  (pad "11" thru_hole circle (at 0 7.62 180) (size 1.7 1.7) (drill 1) (layers "*.Cu" "*.Mask") (remove_unused_layers no)
   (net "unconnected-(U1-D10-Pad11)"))
  (pad "12" thru_hole circle (at 2.54 7.62 180) (size 1.7 1.7) (drill 1) (layers "*.Cu" "*.Mask") (remove_unused_layers no)
   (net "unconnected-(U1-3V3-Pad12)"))
  (pad "13" thru_hole circle (at 5.08 7.62 180) (size 1.7 1.7) (drill 1) (layers "*.Cu" "*.Mask") (remove_unused_layers no)
   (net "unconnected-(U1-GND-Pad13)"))
  (pad "14" thru_hole circle (at 7.62 7.62 180) (size 1.7 1.7) (drill 1) (layers "*.Cu" "*.Mask") (remove_unused_layers no)
   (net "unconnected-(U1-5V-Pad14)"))
  (pad "23" thru_hole circle (at 12.7 0 180) (size 1.7 1.7) (drill 1) (layers "*.Cu" "*.Mask") (remove_unused_layers no) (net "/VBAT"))
  (pad "24" thru_hole circle (at 12.7 5.08 180) (size 1.7 1.7) (drill 1) (layers "*.Cu" "*.Mask") (remove_unused_layers no) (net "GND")))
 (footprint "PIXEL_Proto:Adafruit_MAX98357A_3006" (layer "F.Cu") (at 121.03 125 -90)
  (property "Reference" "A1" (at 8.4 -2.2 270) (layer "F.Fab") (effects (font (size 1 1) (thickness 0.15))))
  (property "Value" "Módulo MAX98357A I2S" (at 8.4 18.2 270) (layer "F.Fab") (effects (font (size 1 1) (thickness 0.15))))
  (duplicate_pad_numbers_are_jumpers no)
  (pad "1" thru_hole rect (at 0 0 270) (size 1.7 1.7) (drill 1) (layers "*.Cu" "*.Mask") (remove_unused_layers no) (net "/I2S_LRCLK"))
  (pad "2" thru_hole circle (at 0 2.54 270) (size 1.7 1.7) (drill 1) (layers "*.Cu" "*.Mask") (remove_unused_layers no) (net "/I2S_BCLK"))
  (pad "3" thru_hole circle (at 0 5.08 270) (size 1.7 1.7) (drill 1) (layers "*.Cu" "*.Mask") (remove_unused_layers no) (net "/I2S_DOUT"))
  (pad "4" thru_hole circle (at 0 7.62 270) (size 1.7 1.7) (drill 1) (layers "*.Cu" "*.Mask") (remove_unused_layers no)
   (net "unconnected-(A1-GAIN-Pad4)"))
  (pad "5" thru_hole circle (at 0 10.16 270) (size 1.7 1.7) (drill 1) (layers "*.Cu" "*.Mask") (remove_unused_layers no)
   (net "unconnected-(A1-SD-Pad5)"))
  (pad "6" thru_hole circle (at 0 12.7 270) (size 1.7 1.7) (drill 1) (layers "*.Cu" "*.Mask") (remove_unused_layers no) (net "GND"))
  (pad "7" thru_hole circle (at 0 15.24 270) (size 1.7 1.7) (drill 1) (layers "*.Cu" "*.Mask") (remove_unused_layers no) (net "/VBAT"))
  (pad "8" thru_hole circle (at 16.3 5.87 270) (size 2 2) (drill 1.2) (layers "*.Cu" "*.Mask") (remove_unused_layers no) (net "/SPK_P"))
  (pad "9" thru_hole circle (at 16.3 9.37 270) (size 2 2) (drill 1.2) (layers "*.Cu" "*.Mask") (remove_unused_layers no) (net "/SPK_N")))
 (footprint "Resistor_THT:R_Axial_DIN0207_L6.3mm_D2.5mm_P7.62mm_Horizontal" (layer "B.Cu") (at 105.79 145.32)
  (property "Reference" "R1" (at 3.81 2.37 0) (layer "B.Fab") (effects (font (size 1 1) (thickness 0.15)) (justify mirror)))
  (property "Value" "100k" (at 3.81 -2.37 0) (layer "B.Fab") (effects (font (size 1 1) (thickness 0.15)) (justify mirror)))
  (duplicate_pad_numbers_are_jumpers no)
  (pad "1" thru_hole circle (at 0 0) (size 1.6 1.6) (drill 0.8) (layers "*.Cu" "*.Mask") (remove_unused_layers no) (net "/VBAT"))
  (pad "2" thru_hole circle (at 7.62 0) (size 1.6 1.6) (drill 0.8) (layers "*.Cu" "*.Mask") (remove_unused_layers no) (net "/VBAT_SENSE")))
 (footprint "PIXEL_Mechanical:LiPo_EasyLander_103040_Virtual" (layer "B.Cu") (at 117.5 120.4 90)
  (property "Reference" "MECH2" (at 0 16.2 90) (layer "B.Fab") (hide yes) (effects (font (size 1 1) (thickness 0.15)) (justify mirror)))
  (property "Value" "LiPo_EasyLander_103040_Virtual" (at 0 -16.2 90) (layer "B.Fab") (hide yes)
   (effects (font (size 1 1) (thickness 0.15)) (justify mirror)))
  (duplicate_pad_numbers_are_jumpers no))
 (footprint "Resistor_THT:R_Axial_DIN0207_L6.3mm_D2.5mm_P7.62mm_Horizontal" (layer "B.Cu") (at 115.95 145.32)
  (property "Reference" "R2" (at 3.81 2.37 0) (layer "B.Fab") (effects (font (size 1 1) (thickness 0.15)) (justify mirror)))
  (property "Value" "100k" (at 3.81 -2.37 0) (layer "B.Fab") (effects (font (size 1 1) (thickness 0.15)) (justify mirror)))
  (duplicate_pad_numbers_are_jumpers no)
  (pad "1" thru_hole circle (at 0 0) (size 1.6 1.6) (drill 0.8) (layers "*.Cu" "*.Mask") (remove_unused_layers no) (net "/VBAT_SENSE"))
  (pad "2" thru_hole circle (at 7.62 0) (size 1.6 1.6) (drill 0.8) (layers "*.Cu" "*.Mask") (remove_unused_layers no) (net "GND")))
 (gr_arc (start 100 100.6) (mid 100.175735 100.175735) (end 100.6 100) (stroke (width 0.1) (type default)) (layer "Edge.Cuts"))
 (gr_line (start 100 149.4) (end 100 100.6) (stroke (width 0.1) (type default)) (layer "Edge.Cuts"))
 (gr_line (start 100.6 100) (end 134.4 100) (stroke (width 0.1) (type default)) (layer "Edge.Cuts"))
 (gr_arc (start 100.6 150) (mid 100.175735 149.824264) (end 100 149.4) (stroke (width 0.1) (type default)) (layer "Edge.Cuts"))
 (gr_arc (start 134.4 100) (mid 134.824264 100.175735) (end 135 100.6) (stroke (width 0.1) (type default)) (layer "Edge.Cuts"))
 (gr_line (start 134.4 150) (end 100.6 150) (stroke (width 0.1) (type default)) (layer "Edge.Cuts"))
 (gr_line (start 135 100.6) (end 135 149.4) (stroke (width 0.1) (type default)) (layer "Edge.Cuts"))
 (gr_arc (start 135 149.4) (mid 134.824264 149.824264) (end 134.4 150) (stroke (width 0.1) (type default)) (layer "Edge.Cuts"))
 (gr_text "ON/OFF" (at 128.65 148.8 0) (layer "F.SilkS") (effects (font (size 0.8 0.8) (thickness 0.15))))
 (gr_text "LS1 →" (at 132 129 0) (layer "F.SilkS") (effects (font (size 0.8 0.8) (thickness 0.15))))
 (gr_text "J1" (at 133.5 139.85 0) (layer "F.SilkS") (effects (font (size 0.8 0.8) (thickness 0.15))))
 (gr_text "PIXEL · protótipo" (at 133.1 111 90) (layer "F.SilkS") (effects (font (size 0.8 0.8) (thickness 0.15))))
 (segment (start 131.19 141.7) (end 128.65 141.7) (width 0.5) (layer "F.Cu") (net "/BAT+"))
 (segment (start 128.65 141.7) (end 128.65 145.32) (width 0.5) (layer "F.Cu") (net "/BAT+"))
 (segment (start 108.33 125) (end 108.33 148.1) (width 0.4) (layer "B.Cu") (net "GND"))
 (segment (start 123.57 145.32) (end 123.57 138) (width 0.4) (layer "B.Cu") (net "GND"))
 (segment (start 108.33 148.1) (end 123.57 148.1) (width 0.4) (layer "B.Cu") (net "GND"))
 (segment (start 123.57 148.1) (end 123.57 145.32) (width 0.4) (layer "B.Cu") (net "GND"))
 (segment (start 107.06 108.49) (end 107.06 123.73) (width 0.4) (layer "B.Cu") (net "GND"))
 (segment (start 107.06 123.73) (end 108.33 125) (width 0.4) (layer "B.Cu") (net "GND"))
 (segment (start 105.79 107.22) (end 107.06 108.49) (width 0.4) (layer "B.Cu") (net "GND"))
 (segment (start 123.57 138) (end 131.19 138) (width 0.4) (layer "B.Cu") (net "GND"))
 (segment (start 105.79 145.32) (end 105.79 147.6) (width 0.5) (layer "F.Cu") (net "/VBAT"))
 (segment (start 126.11 147.6) (end 126.11 145.32) (width 0.5) (layer "F.Cu") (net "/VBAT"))
 (segment (start 105.79 125) (end 105.79 145.32) (width 0.5) (layer "F.Cu") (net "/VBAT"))
 (segment (start 105.79 112.3) (end 105.79 125) (width 0.5) (layer "F.Cu") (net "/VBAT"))
 (segment (start 105.79 147.6) (end 126.11 147.6) (width 0.5) (layer "F.Cu") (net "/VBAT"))
 (segment (start 110.87 119.92) (end 109.6 121.19) (width 0.35) (layer "B.Cu") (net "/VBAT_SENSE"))
 (segment (start 109.6 121.19) (end 109.6 143.4) (width 0.35) (layer "B.Cu") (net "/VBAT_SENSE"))
 (segment (start 113.41 143.4) (end 113.41 145.32) (width 0.35) (layer "B.Cu") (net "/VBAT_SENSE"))
 (segment (start 113.41 145.32) (end 115.95 145.32) (width 0.4) (layer "B.Cu") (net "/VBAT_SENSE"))
 (segment (start 109.6 143.4) (end 113.41 143.4) (width 0.35) (layer "B.Cu") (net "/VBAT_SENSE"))
 (segment (start 115.95 119.92) (end 115.95 125) (width 0.4) (layer "F.Cu") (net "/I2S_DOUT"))
 (segment (start 118.49 119.92) (end 118.49 125) (width 0.4) (layer "F.Cu") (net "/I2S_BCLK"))
 (segment (start 121.03 119.92) (end 121.03 125) (width 0.4) (layer "F.Cu") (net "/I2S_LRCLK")))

